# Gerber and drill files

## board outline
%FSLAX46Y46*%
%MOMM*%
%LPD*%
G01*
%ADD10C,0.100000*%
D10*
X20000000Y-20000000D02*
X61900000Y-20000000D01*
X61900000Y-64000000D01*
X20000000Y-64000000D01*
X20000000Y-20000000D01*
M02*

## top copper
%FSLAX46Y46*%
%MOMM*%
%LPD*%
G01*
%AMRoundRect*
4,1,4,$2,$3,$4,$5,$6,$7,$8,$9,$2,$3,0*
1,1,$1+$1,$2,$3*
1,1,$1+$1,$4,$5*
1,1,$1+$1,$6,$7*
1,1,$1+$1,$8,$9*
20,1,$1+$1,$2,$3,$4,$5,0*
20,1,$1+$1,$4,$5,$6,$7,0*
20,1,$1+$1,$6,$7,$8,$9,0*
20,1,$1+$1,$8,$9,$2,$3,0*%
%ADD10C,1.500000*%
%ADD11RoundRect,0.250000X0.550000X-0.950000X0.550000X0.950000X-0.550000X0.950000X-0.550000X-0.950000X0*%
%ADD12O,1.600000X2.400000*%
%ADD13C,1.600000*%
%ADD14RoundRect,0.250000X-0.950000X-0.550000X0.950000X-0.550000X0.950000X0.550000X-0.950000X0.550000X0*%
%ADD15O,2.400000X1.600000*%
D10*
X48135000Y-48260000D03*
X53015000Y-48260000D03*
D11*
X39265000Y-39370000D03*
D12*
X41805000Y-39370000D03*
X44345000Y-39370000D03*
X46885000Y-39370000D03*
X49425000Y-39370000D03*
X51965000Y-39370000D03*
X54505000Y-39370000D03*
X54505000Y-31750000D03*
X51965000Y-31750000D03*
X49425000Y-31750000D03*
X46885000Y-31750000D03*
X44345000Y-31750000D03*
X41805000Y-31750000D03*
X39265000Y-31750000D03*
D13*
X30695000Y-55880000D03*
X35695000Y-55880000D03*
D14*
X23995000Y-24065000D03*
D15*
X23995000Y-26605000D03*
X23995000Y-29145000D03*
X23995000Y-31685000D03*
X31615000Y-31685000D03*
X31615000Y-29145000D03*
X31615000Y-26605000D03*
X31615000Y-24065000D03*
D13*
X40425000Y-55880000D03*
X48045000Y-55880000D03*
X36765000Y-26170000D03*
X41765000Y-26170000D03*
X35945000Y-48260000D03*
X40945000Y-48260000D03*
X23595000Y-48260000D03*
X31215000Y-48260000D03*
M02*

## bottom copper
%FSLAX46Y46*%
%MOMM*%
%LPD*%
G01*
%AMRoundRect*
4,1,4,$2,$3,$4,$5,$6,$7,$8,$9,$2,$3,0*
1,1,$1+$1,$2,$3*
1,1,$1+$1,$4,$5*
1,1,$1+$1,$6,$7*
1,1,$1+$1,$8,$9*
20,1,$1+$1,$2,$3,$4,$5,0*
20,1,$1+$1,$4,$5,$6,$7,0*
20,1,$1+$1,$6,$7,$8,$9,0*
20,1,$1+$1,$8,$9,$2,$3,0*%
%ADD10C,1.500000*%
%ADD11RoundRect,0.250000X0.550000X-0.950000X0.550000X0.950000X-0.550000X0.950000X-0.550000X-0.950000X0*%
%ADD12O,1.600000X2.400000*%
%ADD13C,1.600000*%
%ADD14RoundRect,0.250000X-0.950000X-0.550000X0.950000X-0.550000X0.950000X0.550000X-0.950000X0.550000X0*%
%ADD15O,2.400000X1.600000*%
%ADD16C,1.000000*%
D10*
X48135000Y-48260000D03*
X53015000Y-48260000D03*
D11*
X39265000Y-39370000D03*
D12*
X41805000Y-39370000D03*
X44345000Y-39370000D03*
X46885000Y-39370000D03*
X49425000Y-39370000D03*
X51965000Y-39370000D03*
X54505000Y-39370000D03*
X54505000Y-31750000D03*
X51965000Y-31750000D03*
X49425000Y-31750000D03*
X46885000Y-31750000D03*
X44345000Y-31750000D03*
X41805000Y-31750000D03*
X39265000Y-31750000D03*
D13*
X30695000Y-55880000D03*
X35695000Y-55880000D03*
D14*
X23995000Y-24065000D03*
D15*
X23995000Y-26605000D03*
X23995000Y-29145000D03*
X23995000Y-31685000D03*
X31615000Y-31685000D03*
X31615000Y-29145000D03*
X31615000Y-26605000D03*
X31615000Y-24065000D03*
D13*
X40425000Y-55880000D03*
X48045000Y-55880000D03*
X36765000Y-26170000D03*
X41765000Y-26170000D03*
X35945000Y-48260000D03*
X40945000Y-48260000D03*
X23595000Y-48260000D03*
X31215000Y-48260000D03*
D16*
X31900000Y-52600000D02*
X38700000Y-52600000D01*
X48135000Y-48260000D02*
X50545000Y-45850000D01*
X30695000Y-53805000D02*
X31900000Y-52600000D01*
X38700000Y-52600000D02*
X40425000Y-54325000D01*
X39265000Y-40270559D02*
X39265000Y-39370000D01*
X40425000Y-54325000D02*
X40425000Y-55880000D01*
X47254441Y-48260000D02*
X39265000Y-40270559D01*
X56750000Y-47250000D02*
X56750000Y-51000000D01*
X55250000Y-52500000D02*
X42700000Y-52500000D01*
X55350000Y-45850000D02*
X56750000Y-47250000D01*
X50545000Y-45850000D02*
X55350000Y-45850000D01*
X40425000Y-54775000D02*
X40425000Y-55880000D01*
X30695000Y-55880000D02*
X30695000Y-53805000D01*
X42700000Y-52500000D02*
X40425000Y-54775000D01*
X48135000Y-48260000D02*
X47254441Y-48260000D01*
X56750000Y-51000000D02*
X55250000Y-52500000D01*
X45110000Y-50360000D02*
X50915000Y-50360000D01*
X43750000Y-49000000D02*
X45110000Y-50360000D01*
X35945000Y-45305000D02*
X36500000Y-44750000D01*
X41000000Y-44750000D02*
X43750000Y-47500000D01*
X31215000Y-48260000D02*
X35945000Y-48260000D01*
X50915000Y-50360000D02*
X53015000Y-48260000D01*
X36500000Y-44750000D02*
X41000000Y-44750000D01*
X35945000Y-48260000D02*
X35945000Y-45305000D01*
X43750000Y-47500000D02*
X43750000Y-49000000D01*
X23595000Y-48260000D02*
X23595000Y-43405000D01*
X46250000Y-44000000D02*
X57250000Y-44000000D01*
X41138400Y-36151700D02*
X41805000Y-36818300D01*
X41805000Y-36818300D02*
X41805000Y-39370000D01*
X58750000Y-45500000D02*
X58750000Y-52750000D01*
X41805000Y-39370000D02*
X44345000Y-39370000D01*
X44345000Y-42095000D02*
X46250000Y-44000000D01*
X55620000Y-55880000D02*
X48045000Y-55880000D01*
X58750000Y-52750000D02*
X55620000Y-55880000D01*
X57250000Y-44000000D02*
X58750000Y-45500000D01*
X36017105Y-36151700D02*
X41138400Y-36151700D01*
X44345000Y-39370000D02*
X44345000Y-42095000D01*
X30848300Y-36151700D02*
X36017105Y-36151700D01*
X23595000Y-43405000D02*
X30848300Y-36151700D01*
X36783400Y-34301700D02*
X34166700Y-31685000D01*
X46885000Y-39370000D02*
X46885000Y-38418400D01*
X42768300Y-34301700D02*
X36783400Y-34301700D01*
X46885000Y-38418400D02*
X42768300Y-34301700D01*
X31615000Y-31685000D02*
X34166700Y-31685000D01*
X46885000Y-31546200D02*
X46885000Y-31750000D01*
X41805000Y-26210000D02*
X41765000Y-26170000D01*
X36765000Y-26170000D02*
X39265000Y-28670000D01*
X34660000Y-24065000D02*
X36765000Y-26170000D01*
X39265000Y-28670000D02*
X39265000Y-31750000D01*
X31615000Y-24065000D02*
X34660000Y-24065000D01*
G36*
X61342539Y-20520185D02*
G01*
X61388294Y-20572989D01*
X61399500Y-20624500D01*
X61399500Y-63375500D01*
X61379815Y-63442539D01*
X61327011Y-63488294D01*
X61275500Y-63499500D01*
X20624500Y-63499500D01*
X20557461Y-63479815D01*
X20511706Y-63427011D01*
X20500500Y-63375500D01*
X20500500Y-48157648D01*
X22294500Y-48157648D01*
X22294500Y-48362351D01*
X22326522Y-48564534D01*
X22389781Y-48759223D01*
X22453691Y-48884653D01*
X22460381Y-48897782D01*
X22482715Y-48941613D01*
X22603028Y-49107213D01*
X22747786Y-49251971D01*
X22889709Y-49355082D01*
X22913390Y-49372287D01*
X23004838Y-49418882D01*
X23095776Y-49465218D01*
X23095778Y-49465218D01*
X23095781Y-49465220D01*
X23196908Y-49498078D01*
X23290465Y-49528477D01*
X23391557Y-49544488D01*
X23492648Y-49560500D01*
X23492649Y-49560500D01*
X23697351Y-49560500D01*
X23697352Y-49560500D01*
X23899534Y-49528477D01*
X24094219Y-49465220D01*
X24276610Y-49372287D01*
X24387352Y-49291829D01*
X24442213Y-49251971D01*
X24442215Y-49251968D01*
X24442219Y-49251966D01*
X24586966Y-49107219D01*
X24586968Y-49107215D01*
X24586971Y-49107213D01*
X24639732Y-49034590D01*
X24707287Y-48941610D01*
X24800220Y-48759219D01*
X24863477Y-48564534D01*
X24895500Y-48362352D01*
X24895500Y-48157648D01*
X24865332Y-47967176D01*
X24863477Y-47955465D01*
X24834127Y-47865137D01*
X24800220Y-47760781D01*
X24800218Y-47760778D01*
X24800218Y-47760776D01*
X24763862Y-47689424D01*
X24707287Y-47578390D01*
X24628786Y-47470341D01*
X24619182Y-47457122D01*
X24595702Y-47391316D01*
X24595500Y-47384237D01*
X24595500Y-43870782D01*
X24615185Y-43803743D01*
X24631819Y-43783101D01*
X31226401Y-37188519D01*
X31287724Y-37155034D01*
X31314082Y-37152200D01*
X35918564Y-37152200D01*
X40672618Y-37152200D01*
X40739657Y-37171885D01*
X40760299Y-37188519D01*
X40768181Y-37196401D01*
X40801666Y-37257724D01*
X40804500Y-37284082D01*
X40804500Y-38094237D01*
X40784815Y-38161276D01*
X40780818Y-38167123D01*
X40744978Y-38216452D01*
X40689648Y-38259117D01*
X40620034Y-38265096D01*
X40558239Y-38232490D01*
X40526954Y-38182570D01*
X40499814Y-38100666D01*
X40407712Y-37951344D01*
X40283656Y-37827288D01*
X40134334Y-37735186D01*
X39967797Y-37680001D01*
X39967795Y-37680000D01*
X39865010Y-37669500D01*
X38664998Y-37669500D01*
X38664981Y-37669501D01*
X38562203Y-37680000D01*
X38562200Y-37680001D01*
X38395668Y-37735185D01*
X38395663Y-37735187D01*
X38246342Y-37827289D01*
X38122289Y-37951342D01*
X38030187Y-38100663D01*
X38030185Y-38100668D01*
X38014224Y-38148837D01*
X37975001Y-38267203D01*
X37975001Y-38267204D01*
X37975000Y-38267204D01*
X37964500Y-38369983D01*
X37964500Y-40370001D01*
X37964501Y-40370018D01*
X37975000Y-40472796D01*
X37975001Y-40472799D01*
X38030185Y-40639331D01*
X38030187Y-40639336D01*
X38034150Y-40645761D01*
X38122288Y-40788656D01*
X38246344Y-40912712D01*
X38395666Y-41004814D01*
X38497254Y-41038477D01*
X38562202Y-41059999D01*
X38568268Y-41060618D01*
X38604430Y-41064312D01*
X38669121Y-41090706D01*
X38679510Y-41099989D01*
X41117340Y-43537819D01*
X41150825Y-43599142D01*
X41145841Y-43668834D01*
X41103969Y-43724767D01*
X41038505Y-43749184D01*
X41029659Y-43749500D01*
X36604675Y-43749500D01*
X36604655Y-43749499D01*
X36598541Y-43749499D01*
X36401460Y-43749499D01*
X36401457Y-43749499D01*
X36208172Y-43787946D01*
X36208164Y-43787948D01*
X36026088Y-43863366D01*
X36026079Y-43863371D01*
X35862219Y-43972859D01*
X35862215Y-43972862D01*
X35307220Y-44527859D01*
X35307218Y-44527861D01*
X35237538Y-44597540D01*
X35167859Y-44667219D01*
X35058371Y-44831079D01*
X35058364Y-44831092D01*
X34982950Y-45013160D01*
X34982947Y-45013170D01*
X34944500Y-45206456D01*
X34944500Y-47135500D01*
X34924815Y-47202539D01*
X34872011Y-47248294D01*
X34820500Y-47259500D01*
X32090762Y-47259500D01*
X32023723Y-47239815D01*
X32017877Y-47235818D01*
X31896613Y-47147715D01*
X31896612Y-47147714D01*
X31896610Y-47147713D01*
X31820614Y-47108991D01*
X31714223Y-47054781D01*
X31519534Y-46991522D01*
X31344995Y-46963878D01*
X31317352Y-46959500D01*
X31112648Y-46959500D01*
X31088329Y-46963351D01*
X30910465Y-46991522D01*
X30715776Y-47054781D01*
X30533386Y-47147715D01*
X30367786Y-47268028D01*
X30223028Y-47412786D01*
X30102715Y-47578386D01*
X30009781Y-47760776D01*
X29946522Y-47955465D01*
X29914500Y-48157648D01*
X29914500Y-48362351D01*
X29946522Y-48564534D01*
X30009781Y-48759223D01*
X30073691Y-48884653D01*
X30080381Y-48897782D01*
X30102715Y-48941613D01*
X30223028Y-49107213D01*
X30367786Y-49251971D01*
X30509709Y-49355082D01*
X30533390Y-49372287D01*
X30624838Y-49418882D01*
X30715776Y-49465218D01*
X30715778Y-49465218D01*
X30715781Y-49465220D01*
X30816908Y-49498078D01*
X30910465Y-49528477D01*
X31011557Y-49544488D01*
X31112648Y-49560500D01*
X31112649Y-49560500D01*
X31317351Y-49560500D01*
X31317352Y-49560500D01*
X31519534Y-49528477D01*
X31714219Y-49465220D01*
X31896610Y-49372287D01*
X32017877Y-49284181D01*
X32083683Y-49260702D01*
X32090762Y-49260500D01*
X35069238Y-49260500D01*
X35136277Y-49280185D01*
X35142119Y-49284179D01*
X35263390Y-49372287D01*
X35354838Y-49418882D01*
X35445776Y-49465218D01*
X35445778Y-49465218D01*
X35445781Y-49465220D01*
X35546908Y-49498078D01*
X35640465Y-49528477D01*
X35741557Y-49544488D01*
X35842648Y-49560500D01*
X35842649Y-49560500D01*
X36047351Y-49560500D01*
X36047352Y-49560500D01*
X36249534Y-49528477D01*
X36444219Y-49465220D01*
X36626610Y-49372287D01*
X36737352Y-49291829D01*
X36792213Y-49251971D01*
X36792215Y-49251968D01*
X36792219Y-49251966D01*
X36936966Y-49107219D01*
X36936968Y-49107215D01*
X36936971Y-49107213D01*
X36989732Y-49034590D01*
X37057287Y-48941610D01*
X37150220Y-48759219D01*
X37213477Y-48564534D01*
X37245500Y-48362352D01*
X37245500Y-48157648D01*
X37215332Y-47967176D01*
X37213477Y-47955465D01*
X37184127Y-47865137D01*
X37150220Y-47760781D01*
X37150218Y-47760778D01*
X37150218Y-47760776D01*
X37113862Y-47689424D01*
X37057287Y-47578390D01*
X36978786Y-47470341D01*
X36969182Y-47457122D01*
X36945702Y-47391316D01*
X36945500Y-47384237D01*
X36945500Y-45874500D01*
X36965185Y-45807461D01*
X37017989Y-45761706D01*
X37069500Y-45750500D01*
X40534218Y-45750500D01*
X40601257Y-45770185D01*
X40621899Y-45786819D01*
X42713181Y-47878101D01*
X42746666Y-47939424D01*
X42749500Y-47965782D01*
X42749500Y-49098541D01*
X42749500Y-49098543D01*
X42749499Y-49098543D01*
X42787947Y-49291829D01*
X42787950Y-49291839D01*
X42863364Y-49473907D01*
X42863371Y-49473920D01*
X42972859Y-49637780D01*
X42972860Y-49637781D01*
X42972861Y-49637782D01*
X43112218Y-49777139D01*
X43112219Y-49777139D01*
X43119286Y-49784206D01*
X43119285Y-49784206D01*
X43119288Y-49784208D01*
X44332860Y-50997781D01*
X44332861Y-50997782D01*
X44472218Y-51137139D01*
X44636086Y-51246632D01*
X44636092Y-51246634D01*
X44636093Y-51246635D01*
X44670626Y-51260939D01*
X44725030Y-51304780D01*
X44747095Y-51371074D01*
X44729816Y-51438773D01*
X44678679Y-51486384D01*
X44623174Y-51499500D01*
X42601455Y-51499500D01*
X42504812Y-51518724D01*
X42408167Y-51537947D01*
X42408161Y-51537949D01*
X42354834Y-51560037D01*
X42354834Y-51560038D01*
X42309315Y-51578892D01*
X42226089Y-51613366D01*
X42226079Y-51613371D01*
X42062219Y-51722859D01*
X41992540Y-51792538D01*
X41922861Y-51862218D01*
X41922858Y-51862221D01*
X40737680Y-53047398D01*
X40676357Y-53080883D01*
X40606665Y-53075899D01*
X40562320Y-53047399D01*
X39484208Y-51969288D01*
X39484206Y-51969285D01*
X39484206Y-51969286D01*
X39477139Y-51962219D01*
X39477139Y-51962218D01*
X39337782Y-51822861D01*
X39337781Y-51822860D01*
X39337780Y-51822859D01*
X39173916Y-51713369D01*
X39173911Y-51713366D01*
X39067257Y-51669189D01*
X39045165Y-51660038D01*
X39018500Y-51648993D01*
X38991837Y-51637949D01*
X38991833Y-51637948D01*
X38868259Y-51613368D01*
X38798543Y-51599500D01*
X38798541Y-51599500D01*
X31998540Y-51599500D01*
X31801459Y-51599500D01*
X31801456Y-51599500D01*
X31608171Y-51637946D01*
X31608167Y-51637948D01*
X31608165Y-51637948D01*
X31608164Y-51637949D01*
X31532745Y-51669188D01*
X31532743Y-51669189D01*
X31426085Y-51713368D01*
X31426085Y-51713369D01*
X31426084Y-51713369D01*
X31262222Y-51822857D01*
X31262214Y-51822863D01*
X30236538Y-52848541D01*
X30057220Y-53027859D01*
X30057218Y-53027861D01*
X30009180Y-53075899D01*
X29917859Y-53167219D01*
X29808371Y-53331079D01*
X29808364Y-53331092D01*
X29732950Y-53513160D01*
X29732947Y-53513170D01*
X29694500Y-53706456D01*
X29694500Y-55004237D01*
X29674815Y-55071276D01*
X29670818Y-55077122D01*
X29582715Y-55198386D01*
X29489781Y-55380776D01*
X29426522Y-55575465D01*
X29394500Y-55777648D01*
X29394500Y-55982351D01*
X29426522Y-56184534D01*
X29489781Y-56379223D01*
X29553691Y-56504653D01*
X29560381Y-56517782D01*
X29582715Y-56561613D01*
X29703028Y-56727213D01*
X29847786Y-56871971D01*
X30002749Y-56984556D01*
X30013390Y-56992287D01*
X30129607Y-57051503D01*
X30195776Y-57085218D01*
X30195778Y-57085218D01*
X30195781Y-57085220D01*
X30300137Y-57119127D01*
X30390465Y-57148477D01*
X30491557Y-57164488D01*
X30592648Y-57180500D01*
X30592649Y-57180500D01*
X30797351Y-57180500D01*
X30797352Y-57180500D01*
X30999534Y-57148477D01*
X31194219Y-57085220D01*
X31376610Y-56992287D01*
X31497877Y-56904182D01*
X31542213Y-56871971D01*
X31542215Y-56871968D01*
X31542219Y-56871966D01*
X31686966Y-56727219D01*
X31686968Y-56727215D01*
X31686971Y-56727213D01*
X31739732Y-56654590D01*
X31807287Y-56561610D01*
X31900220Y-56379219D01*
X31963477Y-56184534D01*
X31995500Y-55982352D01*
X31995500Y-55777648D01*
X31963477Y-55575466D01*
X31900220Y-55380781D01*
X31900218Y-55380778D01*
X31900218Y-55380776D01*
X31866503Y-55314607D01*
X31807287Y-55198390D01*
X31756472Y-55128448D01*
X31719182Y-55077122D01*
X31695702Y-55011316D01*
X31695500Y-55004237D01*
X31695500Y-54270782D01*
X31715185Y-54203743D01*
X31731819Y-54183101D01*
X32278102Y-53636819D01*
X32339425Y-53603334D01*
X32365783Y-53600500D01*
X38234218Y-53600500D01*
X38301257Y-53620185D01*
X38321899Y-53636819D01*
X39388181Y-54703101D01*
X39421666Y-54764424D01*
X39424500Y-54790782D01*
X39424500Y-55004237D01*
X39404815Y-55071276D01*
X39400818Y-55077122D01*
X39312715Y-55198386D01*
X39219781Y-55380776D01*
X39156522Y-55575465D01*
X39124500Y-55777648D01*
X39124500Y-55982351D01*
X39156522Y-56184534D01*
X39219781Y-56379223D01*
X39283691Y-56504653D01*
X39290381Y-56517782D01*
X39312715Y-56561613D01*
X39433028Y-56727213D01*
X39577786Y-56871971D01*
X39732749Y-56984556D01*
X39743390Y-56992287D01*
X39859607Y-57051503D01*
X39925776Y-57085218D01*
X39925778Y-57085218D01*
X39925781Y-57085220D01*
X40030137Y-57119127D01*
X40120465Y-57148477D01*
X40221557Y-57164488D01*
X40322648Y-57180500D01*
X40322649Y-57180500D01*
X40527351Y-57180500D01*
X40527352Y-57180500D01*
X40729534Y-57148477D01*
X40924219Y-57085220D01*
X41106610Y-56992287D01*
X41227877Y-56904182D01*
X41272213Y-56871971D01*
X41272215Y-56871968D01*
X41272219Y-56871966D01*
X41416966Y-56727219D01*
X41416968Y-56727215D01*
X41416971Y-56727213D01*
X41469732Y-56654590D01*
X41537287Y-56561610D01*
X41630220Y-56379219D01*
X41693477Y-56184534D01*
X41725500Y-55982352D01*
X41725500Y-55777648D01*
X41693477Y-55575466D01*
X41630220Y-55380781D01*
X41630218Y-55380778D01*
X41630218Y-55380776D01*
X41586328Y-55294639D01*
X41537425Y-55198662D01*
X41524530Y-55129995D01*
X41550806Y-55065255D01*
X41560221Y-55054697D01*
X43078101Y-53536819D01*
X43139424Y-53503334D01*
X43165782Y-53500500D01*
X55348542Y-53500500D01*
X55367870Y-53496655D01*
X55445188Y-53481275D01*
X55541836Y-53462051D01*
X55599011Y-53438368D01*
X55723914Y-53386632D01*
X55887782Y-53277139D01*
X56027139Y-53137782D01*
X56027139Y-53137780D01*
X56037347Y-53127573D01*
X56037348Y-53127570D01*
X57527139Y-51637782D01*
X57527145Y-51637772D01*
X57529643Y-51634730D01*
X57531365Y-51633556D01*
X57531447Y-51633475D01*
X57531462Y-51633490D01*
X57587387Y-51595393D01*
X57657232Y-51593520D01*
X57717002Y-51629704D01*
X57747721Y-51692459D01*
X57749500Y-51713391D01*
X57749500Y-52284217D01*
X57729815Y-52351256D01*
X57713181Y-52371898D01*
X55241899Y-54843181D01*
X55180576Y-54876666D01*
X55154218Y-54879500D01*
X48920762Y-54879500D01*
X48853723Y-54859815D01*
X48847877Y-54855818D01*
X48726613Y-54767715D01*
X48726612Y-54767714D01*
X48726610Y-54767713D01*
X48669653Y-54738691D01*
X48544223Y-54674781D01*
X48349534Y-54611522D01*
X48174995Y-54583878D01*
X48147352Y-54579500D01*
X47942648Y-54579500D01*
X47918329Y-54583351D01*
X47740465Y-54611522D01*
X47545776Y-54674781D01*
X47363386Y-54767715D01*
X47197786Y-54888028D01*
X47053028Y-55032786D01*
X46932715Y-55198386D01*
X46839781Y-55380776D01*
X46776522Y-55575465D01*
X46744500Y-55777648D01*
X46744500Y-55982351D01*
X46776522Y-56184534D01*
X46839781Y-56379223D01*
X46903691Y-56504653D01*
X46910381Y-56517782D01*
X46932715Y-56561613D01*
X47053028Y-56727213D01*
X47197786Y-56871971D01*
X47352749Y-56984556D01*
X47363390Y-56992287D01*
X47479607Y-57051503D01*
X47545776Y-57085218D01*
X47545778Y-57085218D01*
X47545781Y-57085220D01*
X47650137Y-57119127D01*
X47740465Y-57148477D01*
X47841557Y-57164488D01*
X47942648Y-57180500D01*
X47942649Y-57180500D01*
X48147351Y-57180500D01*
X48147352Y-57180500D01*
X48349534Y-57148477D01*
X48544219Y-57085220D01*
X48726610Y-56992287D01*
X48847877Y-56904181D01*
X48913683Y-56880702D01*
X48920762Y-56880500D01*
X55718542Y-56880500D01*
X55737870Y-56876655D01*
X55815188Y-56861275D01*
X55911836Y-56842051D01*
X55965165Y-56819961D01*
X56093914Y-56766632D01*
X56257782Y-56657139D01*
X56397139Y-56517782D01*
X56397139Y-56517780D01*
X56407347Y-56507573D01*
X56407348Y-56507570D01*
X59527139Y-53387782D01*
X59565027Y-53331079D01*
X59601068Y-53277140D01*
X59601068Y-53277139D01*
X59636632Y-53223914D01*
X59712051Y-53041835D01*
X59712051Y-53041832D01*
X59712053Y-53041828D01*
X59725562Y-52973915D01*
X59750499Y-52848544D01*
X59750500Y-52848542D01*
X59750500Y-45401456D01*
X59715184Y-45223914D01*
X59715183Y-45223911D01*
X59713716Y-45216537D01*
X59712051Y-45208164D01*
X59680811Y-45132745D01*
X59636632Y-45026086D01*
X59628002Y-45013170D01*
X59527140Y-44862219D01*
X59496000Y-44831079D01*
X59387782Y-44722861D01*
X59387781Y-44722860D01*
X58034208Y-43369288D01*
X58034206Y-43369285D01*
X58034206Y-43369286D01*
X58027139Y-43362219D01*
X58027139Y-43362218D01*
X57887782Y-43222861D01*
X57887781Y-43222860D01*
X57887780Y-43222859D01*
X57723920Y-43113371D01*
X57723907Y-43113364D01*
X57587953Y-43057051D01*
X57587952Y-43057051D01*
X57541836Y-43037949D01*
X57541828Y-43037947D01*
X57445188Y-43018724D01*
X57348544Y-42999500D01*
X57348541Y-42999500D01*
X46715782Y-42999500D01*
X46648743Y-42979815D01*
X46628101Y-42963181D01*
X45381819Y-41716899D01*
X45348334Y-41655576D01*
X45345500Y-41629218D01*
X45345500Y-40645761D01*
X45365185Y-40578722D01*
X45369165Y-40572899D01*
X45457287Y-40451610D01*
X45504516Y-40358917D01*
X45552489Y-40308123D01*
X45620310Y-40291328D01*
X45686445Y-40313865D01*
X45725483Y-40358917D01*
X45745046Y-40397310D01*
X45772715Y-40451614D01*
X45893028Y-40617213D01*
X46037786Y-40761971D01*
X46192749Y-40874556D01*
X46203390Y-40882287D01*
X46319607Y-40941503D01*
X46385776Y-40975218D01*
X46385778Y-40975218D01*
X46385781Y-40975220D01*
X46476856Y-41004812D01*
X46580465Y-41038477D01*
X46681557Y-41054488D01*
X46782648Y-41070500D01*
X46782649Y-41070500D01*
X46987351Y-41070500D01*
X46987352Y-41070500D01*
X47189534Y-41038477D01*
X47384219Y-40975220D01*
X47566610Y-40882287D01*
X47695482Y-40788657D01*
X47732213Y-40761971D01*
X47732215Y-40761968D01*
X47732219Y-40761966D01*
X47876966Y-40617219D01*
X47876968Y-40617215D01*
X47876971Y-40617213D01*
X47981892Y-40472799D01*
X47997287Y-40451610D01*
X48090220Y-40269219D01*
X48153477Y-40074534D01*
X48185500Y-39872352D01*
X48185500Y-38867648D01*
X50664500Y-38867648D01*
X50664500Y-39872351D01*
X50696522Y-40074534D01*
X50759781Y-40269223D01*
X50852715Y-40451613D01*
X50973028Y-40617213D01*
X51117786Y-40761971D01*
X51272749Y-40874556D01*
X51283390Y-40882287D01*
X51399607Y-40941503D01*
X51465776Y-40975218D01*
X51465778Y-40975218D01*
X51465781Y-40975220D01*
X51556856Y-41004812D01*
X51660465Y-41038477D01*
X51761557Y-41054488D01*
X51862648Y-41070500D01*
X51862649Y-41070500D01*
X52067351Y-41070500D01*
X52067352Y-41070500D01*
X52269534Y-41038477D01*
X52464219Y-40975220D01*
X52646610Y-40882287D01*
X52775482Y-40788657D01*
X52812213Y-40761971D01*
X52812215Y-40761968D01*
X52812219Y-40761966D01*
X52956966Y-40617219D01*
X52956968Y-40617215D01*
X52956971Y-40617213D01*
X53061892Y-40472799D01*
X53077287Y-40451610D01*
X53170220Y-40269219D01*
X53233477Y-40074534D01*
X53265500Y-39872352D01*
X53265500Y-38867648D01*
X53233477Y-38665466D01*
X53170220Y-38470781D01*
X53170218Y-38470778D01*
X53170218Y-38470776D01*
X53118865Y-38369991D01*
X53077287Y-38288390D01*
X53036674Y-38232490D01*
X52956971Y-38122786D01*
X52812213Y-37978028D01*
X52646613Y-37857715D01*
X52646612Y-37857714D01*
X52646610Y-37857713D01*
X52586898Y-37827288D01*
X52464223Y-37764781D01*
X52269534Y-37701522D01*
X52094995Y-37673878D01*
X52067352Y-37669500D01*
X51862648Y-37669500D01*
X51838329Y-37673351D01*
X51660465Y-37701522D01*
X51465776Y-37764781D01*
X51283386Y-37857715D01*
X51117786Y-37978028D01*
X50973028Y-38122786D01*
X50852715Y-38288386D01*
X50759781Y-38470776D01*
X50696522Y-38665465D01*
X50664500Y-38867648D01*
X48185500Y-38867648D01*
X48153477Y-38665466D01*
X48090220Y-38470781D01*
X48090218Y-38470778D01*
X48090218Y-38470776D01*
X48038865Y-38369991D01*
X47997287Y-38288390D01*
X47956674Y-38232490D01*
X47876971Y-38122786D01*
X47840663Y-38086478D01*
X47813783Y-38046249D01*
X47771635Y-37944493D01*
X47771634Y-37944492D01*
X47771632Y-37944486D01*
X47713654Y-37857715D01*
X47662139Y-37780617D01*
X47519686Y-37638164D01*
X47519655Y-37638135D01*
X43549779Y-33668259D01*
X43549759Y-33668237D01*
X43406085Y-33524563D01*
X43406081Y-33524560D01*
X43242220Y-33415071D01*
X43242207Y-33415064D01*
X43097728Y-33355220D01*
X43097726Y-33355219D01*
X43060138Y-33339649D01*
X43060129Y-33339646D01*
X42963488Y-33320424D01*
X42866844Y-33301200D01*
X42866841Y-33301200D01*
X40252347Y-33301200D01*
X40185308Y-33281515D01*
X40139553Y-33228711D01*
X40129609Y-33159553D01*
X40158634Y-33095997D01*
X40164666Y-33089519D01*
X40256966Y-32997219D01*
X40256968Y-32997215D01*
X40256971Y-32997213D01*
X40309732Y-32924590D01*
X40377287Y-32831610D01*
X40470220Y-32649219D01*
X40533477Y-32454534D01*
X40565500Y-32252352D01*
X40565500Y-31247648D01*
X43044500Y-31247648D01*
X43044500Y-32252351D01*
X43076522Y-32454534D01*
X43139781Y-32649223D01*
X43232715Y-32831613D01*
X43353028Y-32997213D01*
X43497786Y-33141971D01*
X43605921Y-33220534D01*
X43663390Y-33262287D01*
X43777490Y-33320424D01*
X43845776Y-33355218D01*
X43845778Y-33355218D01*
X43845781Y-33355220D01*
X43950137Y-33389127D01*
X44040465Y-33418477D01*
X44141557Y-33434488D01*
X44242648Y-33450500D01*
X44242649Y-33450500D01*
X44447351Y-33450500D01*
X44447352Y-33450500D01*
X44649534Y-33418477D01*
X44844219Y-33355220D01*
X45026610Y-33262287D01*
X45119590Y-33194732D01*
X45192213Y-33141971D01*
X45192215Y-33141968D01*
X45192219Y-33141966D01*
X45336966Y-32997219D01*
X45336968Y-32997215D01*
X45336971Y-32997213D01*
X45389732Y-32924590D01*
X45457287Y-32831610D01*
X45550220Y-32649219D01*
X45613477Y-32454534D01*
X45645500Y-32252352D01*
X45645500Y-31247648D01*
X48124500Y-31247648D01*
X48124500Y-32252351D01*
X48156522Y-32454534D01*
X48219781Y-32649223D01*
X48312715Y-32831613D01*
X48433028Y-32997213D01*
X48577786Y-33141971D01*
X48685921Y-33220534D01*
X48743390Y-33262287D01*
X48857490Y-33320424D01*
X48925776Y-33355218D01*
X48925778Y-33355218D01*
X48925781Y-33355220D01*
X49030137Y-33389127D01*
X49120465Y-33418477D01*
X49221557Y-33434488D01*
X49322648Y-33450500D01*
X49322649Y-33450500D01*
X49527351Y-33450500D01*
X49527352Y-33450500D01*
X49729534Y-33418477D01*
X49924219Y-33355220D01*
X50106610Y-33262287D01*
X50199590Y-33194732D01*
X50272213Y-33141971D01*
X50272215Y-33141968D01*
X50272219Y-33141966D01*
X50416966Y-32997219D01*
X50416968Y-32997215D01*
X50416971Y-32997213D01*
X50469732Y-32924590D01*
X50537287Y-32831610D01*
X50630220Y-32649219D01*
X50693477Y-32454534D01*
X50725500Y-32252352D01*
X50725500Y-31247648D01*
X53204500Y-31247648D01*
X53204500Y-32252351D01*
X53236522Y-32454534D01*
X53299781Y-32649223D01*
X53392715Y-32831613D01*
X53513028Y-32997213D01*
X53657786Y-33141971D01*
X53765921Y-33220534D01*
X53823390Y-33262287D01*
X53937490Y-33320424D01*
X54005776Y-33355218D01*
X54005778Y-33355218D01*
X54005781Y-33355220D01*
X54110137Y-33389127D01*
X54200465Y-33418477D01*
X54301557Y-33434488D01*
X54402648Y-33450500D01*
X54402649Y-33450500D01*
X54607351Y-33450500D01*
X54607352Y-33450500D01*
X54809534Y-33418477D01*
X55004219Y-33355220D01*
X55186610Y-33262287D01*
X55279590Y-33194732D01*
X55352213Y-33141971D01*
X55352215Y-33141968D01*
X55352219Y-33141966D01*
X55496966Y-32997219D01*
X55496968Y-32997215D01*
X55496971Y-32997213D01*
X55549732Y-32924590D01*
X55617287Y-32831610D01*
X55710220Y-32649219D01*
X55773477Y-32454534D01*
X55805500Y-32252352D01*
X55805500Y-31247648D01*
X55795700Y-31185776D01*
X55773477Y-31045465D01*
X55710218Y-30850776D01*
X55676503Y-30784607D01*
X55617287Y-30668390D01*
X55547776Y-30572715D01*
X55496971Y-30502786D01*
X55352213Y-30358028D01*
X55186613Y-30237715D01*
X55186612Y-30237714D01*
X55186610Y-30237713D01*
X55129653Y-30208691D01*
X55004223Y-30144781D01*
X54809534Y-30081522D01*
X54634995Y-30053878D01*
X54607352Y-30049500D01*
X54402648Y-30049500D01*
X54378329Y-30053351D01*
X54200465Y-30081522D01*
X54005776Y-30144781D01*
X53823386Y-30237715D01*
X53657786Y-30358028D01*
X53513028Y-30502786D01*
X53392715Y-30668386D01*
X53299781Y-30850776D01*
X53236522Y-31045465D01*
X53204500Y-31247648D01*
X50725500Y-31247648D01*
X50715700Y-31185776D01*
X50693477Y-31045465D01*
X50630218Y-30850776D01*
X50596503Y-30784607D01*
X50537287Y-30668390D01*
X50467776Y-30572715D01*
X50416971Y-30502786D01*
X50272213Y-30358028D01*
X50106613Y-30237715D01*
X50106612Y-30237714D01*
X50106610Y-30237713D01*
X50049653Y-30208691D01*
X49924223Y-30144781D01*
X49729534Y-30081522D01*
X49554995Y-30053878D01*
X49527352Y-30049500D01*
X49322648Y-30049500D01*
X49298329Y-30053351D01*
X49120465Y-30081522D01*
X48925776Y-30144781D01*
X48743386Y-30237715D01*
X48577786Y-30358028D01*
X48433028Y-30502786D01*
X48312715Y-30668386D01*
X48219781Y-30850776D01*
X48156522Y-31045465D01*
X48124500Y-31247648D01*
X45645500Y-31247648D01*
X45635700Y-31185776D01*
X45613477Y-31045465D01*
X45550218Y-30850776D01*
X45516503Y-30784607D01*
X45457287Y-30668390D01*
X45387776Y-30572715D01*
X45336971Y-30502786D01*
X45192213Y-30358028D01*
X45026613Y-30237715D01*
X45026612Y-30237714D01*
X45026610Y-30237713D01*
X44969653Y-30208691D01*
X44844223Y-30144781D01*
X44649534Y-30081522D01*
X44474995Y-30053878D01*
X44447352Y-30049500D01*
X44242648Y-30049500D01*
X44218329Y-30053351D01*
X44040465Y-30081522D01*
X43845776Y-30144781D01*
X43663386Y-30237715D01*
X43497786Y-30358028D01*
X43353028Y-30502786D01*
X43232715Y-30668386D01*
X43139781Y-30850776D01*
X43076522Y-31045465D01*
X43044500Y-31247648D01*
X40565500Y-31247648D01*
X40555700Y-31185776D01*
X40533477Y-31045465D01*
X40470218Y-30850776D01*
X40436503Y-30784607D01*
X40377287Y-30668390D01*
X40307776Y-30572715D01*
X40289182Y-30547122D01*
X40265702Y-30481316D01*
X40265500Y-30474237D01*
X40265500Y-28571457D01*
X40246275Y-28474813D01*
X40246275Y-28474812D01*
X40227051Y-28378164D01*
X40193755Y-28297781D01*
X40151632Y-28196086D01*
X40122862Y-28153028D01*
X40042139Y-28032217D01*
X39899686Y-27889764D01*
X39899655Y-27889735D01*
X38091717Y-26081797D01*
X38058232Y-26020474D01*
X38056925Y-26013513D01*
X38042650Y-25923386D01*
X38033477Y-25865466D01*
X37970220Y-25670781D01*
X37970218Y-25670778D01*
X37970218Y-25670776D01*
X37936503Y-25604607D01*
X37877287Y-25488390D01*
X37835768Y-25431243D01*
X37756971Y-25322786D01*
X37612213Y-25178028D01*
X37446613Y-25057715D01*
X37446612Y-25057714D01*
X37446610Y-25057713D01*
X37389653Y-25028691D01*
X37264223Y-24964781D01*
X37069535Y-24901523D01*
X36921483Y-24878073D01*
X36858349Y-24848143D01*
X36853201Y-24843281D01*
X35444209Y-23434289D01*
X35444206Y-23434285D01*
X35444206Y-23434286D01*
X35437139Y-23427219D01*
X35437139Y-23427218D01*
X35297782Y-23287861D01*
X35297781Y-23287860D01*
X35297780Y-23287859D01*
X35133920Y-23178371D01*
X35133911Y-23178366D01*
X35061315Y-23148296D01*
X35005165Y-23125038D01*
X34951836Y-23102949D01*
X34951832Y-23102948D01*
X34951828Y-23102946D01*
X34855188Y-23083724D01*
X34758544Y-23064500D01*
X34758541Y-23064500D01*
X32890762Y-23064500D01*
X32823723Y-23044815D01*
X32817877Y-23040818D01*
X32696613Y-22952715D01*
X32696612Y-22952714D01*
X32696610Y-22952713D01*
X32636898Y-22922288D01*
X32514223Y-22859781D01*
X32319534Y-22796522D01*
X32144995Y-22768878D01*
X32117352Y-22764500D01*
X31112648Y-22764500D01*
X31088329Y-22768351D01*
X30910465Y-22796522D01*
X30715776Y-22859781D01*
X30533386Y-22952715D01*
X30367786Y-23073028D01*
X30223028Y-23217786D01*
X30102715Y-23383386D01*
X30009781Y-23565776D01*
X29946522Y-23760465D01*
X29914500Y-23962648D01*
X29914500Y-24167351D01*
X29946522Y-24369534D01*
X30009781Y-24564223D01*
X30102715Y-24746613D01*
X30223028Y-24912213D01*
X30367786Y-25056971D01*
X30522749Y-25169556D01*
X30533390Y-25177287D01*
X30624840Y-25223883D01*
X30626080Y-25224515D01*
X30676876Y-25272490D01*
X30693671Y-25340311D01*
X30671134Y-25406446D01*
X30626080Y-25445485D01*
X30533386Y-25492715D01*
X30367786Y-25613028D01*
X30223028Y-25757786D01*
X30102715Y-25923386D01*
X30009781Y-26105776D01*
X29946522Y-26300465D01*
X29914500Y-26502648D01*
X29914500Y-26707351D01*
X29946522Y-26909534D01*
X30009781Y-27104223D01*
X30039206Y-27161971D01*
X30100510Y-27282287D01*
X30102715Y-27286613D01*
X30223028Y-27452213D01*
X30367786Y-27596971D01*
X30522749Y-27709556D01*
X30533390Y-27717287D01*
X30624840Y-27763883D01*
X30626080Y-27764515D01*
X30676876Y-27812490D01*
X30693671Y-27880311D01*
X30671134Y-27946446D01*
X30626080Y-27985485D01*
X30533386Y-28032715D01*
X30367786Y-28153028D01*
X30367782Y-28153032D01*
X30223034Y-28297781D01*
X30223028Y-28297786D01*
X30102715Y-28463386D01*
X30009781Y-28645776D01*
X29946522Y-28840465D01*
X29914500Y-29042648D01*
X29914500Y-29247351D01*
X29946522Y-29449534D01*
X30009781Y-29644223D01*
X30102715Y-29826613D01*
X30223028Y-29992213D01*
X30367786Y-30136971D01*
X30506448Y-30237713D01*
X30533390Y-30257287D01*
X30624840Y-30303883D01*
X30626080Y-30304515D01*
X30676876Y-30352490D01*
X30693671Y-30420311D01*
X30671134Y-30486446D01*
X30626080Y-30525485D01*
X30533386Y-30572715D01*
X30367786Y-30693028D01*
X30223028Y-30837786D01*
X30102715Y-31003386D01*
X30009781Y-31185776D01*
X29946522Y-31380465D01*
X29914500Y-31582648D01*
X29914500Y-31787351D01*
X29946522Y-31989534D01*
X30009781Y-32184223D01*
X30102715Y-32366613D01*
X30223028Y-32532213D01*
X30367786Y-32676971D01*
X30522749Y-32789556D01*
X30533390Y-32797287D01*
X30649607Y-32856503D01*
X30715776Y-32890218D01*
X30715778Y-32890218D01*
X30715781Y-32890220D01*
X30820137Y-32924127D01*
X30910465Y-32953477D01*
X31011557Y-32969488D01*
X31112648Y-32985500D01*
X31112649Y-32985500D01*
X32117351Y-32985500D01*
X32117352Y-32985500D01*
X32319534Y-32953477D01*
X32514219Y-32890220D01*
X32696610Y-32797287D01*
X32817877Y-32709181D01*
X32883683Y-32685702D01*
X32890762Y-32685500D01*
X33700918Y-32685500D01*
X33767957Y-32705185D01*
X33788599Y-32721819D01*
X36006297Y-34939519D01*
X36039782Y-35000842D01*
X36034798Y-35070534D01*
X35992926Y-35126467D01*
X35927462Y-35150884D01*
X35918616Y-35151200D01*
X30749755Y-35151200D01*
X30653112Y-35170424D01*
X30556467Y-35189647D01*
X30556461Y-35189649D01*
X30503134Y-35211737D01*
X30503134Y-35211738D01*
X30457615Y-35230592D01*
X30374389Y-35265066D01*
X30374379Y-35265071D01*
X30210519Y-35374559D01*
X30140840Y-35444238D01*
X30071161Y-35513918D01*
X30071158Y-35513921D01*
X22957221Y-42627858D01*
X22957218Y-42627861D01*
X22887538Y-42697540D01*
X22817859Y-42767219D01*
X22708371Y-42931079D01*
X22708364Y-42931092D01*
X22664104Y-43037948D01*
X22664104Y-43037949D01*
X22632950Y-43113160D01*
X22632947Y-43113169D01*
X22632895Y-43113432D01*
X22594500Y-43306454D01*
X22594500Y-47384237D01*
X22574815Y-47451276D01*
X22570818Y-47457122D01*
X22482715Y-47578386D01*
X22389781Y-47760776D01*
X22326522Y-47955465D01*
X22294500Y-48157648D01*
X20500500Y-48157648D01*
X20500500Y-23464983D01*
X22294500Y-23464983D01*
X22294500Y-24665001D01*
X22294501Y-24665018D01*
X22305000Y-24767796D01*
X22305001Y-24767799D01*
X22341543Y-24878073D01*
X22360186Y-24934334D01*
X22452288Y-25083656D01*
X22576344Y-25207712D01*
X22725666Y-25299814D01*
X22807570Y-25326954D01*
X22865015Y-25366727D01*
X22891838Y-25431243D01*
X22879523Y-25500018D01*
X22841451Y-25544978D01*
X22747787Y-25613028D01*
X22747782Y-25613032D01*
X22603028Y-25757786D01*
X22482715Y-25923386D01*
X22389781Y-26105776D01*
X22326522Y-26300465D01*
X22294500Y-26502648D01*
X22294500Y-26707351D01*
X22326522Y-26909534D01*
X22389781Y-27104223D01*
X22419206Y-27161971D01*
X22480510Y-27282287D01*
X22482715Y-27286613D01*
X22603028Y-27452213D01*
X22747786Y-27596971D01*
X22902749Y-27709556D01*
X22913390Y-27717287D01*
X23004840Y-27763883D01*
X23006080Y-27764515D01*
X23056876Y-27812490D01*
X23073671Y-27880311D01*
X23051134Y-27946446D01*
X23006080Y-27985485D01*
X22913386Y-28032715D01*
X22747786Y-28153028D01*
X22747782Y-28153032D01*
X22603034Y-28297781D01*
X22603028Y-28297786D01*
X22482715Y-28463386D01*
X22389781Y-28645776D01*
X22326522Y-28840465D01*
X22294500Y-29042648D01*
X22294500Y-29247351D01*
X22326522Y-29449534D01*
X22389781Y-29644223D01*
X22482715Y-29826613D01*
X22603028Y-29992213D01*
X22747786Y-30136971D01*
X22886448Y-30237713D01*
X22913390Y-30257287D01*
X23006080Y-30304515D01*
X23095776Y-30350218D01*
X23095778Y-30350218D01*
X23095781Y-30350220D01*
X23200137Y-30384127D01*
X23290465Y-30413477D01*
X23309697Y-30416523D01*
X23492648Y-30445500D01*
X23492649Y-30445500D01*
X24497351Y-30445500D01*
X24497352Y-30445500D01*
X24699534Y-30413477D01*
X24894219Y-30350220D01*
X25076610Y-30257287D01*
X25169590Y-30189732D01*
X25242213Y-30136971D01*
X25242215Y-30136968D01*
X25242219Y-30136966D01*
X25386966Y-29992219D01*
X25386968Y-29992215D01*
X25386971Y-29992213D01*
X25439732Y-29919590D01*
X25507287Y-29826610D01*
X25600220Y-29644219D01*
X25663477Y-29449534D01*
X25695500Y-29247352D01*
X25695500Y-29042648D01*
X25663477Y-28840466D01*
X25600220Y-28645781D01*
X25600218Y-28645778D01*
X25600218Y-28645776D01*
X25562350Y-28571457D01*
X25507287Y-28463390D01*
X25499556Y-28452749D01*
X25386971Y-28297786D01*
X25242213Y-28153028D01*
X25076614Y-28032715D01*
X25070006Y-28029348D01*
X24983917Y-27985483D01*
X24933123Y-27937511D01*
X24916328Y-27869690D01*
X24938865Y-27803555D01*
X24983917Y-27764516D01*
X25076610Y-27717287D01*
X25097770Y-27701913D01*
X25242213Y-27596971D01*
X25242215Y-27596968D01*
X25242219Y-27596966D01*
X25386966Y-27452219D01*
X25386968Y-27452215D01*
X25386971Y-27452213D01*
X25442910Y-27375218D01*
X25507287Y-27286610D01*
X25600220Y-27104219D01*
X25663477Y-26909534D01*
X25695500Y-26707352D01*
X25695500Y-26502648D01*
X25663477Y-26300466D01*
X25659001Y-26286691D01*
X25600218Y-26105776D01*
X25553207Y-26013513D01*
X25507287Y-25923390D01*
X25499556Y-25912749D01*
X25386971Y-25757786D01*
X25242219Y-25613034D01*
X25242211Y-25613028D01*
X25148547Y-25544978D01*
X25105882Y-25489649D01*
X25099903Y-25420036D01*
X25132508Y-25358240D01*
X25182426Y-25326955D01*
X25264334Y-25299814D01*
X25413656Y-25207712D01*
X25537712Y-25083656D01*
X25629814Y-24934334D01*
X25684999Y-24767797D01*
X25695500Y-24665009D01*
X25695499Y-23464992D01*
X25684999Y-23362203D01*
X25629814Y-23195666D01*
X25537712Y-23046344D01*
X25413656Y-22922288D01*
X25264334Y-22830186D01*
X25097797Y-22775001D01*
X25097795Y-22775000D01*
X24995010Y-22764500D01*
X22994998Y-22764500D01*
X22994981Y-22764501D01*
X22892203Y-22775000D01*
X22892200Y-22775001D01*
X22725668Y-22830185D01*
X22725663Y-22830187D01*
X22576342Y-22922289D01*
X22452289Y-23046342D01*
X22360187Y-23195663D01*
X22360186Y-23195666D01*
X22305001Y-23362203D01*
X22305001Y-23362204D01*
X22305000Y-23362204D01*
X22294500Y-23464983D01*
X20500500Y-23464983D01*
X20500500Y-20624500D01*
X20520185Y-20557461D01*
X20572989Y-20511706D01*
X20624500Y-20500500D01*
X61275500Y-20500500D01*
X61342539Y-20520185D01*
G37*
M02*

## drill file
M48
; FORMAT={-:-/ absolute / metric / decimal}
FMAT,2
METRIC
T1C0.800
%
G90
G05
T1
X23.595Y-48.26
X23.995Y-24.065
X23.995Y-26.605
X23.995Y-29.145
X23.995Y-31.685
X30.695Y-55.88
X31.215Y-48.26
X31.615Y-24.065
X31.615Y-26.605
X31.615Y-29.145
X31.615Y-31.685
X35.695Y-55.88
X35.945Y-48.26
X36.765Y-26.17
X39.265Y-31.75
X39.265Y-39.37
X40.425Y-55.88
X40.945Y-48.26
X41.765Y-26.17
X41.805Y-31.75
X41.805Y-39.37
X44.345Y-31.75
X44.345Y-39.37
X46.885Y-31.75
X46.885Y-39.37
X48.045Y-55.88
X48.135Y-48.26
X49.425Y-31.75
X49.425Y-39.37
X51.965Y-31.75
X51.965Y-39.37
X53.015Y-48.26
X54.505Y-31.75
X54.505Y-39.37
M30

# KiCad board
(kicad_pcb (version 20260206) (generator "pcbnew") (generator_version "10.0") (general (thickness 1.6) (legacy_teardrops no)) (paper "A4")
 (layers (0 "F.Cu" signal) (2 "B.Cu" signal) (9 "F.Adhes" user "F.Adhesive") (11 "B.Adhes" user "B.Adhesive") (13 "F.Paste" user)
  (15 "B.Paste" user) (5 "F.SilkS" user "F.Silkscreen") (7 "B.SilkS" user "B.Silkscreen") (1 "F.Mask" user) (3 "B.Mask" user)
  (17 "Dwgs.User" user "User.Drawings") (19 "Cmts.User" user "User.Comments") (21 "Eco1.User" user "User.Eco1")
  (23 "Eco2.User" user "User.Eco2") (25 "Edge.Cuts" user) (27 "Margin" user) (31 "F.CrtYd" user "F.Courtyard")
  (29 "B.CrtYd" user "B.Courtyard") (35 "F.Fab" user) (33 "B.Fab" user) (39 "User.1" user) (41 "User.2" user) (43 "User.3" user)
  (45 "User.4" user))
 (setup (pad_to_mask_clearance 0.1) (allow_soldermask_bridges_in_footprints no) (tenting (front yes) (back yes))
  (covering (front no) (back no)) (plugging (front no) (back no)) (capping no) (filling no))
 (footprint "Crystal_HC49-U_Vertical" (layer "F.Cu") (at 48.135 48.26)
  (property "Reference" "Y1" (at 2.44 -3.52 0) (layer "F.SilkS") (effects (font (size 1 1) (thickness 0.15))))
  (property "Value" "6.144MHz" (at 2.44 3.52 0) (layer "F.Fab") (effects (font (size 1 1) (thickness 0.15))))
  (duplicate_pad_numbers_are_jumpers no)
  (pad "1" thru_hole circle (at 0 0) (size 1.5 1.5) (drill 0.8) (layers "*.Cu" "*.Mask") (remove_unused_layers no) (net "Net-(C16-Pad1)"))
  (pad "2" thru_hole circle (at 4.88 0) (size 1.5 1.5) (drill 0.8) (layers "*.Cu" "*.Mask") (remove_unused_layers no) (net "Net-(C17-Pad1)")))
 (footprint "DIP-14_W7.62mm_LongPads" (layer "F.Cu") (at 39.265 39.37 90)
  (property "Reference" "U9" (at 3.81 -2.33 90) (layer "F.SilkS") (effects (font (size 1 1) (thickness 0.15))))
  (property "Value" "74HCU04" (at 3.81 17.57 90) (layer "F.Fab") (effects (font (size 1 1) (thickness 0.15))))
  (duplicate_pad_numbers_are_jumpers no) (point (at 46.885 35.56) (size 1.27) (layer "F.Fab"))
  (pad "1" thru_hole roundrect (at 0 0 90) (size 2.4 1.6) (drill 0.8) (layers "*.Cu" "*.Mask") (remove_unused_layers no)
   (roundrect_rratio 0.15625) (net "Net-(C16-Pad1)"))
  (pad "2" thru_hole oval (at 0 2.54 90) (size 2.4 1.6) (drill 0.8) (layers "*.Cu" "*.Mask") (remove_unused_layers no)
   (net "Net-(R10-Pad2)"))
  (pad "3" thru_hole oval (at 0 5.08 90) (size 2.4 1.6) (drill 0.8) (layers "*.Cu" "*.Mask") (remove_unused_layers no)
   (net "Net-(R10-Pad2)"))
  (pad "4" thru_hole oval (at 0 7.62 90) (size 2.4 1.6) (drill 0.8) (layers "*.Cu" "*.Mask") (remove_unused_layers no)
   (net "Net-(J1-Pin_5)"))
  (pad "5" thru_hole oval (at 0 10.16 90) (size 2.4 1.6) (drill 0.8) (layers "*.Cu" "*.Mask") (remove_unused_layers no) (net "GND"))
  (pad "6" thru_hole oval (at 0 12.7 90) (size 2.4 1.6) (drill 0.8) (layers "*.Cu" "*.Mask") (remove_unused_layers no))
  (pad "7" thru_hole oval (at 0 15.24 90) (size 2.4 1.6) (drill 0.8) (layers "*.Cu" "*.Mask") (remove_unused_layers no) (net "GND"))
  (pad "8" thru_hole oval (at 7.62 15.24 90) (size 2.4 1.6) (drill 0.8) (layers "*.Cu" "*.Mask") (remove_unused_layers no))
  (pad "9" thru_hole oval (at 7.62 12.7 90) (size 2.4 1.6) (drill 0.8) (layers "*.Cu" "*.Mask") (remove_unused_layers no) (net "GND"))
  (pad "10" thru_hole oval (at 7.62 10.16 90) (size 2.4 1.6) (drill 0.8) (layers "*.Cu" "*.Mask") (remove_unused_layers no))
  (pad "11" thru_hole oval (at 7.62 7.62 90) (size 2.4 1.6) (drill 0.8) (layers "*.Cu" "*.Mask") (remove_unused_layers no) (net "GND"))
  (pad "12" thru_hole oval (at 7.62 5.08 90) (size 2.4 1.6) (drill 0.8) (layers "*.Cu" "*.Mask") (remove_unused_layers no))
  (pad "13" thru_hole oval (at 7.62 2.54 90) (size 2.4 1.6) (drill 0.8) (layers "*.Cu" "*.Mask") (remove_unused_layers no) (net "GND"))
  (pad "14" thru_hole oval (at 7.62 0 90) (size 2.4 1.6) (drill 0.8) (layers "*.Cu" "*.Mask") (remove_unused_layers no) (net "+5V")))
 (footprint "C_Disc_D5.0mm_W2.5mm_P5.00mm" (layer "F.Cu") (at 30.695 55.88)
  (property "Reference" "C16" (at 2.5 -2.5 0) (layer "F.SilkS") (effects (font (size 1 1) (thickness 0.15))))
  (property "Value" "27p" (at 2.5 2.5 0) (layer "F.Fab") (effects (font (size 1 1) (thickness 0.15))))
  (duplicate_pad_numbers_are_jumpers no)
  (pad "1" thru_hole circle (at 0 0) (size 1.6 1.6) (drill 0.8) (layers "*.Cu" "*.Mask") (remove_unused_layers no) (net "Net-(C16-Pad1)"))
  (pad "2" thru_hole circle (at 5 0) (size 1.6 1.6) (drill 0.8) (layers "*.Cu" "*.Mask") (remove_unused_layers no) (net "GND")))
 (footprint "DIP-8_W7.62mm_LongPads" (layer "F.Cu") (at 23.995 24.065)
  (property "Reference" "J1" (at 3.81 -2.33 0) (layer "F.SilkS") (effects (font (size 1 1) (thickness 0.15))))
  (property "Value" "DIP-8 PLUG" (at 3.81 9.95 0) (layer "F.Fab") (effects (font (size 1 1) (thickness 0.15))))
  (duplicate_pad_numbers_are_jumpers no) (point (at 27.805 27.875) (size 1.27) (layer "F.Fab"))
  (pad "1" thru_hole roundrect (at 0 0) (size 2.4 1.6) (drill 0.8) (layers "*.Cu" "*.Mask") (remove_unused_layers no)
   (roundrect_rratio 0.15625))
  (pad "2" thru_hole oval (at 0 2.54) (size 2.4 1.6) (drill 0.8) (layers "*.Cu" "*.Mask") (remove_unused_layers no))
  (pad "3" thru_hole oval (at 0 5.08) (size 2.4 1.6) (drill 0.8) (layers "*.Cu" "*.Mask") (remove_unused_layers no))
  (pad "4" thru_hole oval (at 0 7.62) (size 2.4 1.6) (drill 0.8) (layers "*.Cu" "*.Mask") (remove_unused_layers no) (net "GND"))
  (pad "5" thru_hole oval (at 7.62 7.62) (size 2.4 1.6) (drill 0.8) (layers "*.Cu" "*.Mask") (remove_unused_layers no)
   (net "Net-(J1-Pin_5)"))
  (pad "6" thru_hole oval (at 7.62 5.08) (size 2.4 1.6) (drill 0.8) (layers "*.Cu" "*.Mask") (remove_unused_layers no))
  (pad "7" thru_hole oval (at 7.62 2.54) (size 2.4 1.6) (drill 0.8) (layers "*.Cu" "*.Mask") (remove_unused_layers no))
  (pad "8" thru_hole oval (at 7.62 0) (size 2.4 1.6) (drill 0.8) (layers "*.Cu" "*.Mask") (remove_unused_layers no) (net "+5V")))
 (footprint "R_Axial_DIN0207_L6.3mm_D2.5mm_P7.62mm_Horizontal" (layer "F.Cu") (at 40.425 55.88)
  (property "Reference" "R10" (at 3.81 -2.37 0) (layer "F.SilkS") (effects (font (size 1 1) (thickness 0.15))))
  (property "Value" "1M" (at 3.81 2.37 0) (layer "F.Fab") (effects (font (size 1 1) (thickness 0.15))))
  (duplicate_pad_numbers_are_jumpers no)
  (pad "1" thru_hole circle (at 0 0) (size 1.6 1.6) (drill 0.8) (layers "*.Cu" "*.Mask") (remove_unused_layers no) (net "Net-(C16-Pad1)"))
  (pad "2" thru_hole circle (at 7.62 0) (size 1.6 1.6) (drill 0.8) (layers "*.Cu" "*.Mask") (remove_unused_layers no) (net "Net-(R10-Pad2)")))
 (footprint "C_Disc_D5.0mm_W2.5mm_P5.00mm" (layer "F.Cu") (at 36.765 26.17)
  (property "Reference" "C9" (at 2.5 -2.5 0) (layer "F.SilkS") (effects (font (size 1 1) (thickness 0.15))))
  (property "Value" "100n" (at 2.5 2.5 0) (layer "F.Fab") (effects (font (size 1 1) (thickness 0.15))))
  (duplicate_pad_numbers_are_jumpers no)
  (pad "1" thru_hole circle (at 0 0) (size 1.6 1.6) (drill 0.8) (layers "*.Cu" "*.Mask") (remove_unused_layers no) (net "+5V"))
  (pad "2" thru_hole circle (at 5 0) (size 1.6 1.6) (drill 0.8) (layers "*.Cu" "*.Mask") (remove_unused_layers no) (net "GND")))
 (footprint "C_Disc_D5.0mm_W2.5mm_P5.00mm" (layer "F.Cu") (at 35.945 48.26)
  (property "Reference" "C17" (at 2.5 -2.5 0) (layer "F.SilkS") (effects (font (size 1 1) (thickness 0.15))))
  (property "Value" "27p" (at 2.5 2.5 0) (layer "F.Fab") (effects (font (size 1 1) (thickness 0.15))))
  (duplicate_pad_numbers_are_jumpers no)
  (pad "1" thru_hole circle (at 0 0) (size 1.6 1.6) (drill 0.8) (layers "*.Cu" "*.Mask") (remove_unused_layers no) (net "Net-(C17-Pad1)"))
  (pad "2" thru_hole circle (at 5 0) (size 1.6 1.6) (drill 0.8) (layers "*.Cu" "*.Mask") (remove_unused_layers no) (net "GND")))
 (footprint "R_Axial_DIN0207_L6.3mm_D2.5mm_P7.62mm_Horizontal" (layer "F.Cu") (at 23.595 48.26)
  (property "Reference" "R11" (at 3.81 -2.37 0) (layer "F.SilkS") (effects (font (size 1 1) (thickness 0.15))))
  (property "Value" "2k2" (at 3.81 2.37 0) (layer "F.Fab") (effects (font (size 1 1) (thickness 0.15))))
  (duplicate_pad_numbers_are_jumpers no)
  (pad "1" thru_hole circle (at 0 0) (size 1.6 1.6) (drill 0.8) (layers "*.Cu" "*.Mask") (remove_unused_layers no) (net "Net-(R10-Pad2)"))
  (pad "2" thru_hole circle (at 7.62 0) (size 1.6 1.6) (drill 0.8) (layers "*.Cu" "*.Mask") (remove_unused_layers no) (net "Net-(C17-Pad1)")))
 (gr_rect (start 20 20) (end 61.9 64) (stroke (width 0.1) (type default)) (fill no) (layer "Edge.Cuts"))
 (segment (start 31.9 52.6) (end 38.7 52.6) (width 1) (layer "B.Cu") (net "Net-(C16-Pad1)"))
 (segment (start 48.135 48.26) (end 50.545 45.85) (width 1) (layer "B.Cu") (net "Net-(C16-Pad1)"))
 (segment (start 30.695 53.805) (end 31.9 52.6) (width 1) (layer "B.Cu") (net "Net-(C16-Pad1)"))
 (segment (start 38.7 52.6) (end 40.425 54.325) (width 1) (layer "B.Cu") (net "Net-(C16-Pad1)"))
 (segment (start 39.265 40.270559) (end 39.265 39.37) (width 1) (layer "B.Cu") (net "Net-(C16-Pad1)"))
 (segment (start 40.425 54.325) (end 40.425 55.88) (width 1) (layer "B.Cu") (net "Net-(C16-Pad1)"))
 (segment (start 47.254441 48.26) (end 39.265 40.270559) (width 1) (layer "B.Cu") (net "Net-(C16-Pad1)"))
 (segment (start 56.75 47.25) (end 56.75 51) (width 1) (layer "B.Cu") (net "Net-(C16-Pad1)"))
 (segment (start 55.25 52.5) (end 42.7 52.5) (width 1) (layer "B.Cu") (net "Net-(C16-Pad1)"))
 (segment (start 55.35 45.85) (end 56.75 47.25) (width 1) (layer "B.Cu") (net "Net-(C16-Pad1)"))
 (segment (start 50.545 45.85) (end 55.35 45.85) (width 1) (layer "B.Cu") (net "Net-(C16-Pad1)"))
 (segment (start 40.425 54.775) (end 40.425 55.88) (width 1) (layer "B.Cu") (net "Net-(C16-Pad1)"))
 (segment (start 30.695 55.88) (end 30.695 53.805) (width 1) (layer "B.Cu") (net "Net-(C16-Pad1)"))
 (segment (start 42.7 52.5) (end 40.425 54.775) (width 1) (layer "B.Cu") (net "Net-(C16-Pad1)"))
 (segment (start 48.135 48.26) (end 47.254441 48.26) (width 1) (layer "B.Cu") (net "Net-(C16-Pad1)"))
 (segment (start 56.75 51) (end 55.25 52.5) (width 1) (layer "B.Cu") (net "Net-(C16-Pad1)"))
 (segment (start 45.11 50.36) (end 50.915 50.36) (width 1) (layer "B.Cu") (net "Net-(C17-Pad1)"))
 (segment (start 43.75 49) (end 45.11 50.36) (width 1) (layer "B.Cu") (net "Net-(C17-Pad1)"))
 (segment (start 35.945 45.305) (end 36.5 44.75) (width 1) (layer "B.Cu") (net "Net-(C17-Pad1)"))
 (segment (start 41 44.75) (end 43.75 47.5) (width 1) (layer "B.Cu") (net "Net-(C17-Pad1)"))
 (segment (start 31.215 48.26) (end 35.945 48.26) (width 1) (layer "B.Cu") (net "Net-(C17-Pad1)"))
 (segment (start 50.915 50.36) (end 53.015 48.26) (width 1) (layer "B.Cu") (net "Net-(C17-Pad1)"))
 (segment (start 36.5 44.75) (end 41 44.75) (width 1) (layer "B.Cu") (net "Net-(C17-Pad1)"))
 (segment (start 35.945 48.26) (end 35.945 45.305) (width 1) (layer "B.Cu") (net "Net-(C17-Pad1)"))
 (segment (start 43.75 47.5) (end 43.75 49) (width 1) (layer "B.Cu") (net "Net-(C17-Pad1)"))
 (segment (start 23.595 48.26) (end 23.595 43.405) (width 1) (layer "B.Cu") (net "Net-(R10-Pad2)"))
 (segment (start 46.25 44) (end 57.25 44) (width 1) (layer "B.Cu") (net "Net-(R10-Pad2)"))
 (segment (start 41.1384 36.1517) (end 41.805 36.8183) (width 1) (layer "B.Cu") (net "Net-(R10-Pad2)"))
 (segment (start 41.805 36.8183) (end 41.805 39.37) (width 1) (layer "B.Cu") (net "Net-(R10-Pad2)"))
 (segment (start 58.75 45.5) (end 58.75 52.75) (width 1) (layer "B.Cu") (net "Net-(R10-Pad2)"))
 (segment (start 41.805 39.37) (end 44.345 39.37) (width 1) (layer "B.Cu") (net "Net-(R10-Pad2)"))
 (segment (start 44.345 42.095) (end 46.25 44) (width 1) (layer "B.Cu") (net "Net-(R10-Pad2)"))
 (segment (start 55.62 55.88) (end 48.045 55.88) (width 1) (layer "B.Cu") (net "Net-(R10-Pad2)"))
 (segment (start 58.75 52.75) (end 55.62 55.88) (width 1) (layer "B.Cu") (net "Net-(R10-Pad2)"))
 (segment (start 57.25 44) (end 58.75 45.5) (width 1) (layer "B.Cu") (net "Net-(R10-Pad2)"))
 (segment (start 36.017105 36.1517) (end 41.1384 36.1517) (width 1) (layer "B.Cu") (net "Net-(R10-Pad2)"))
 (segment (start 44.345 39.37) (end 44.345 42.095) (width 1) (layer "B.Cu") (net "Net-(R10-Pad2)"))
 (segment (start 30.8483 36.1517) (end 36.017105 36.1517) (width 1) (layer "B.Cu") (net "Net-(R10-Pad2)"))
 (segment (start 23.595 43.405) (end 30.8483 36.1517) (width 1) (layer "B.Cu") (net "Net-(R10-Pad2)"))
 (segment (start 36.7834 34.3017) (end 34.1667 31.685) (width 1) (layer "B.Cu") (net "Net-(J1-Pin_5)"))
 (segment (start 46.885 39.37) (end 46.885 38.4184) (width 1) (layer "B.Cu") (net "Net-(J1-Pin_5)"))
 (segment (start 42.7683 34.3017) (end 36.7834 34.3017) (width 1) (layer "B.Cu") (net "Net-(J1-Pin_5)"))
 (segment (start 46.885 38.4184) (end 42.7683 34.3017) (width 1) (layer "B.Cu") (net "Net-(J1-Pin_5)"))
 (segment (start 31.615 31.685) (end 34.1667 31.685) (width 1) (layer "B.Cu") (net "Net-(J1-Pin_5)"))
 (segment (start 46.885 31.5462) (end 46.885 31.75) (width 1) (layer "B.Cu") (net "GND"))
 (segment (start 41.805 26.21) (end 41.765 26.17) (width 1) (layer "B.Cu") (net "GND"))
 (segment (start 36.765 26.17) (end 39.265 28.67) (width 1) (layer "B.Cu") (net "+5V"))
 (segment (start 34.66 24.065) (end 36.765 26.17) (width 1) (layer "B.Cu") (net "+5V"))
 (segment (start 39.265 28.67) (end 39.265 31.75) (width 1) (layer "B.Cu") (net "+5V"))
 (segment (start 31.615 24.065) (end 34.66 24.065) (width 1) (layer "B.Cu") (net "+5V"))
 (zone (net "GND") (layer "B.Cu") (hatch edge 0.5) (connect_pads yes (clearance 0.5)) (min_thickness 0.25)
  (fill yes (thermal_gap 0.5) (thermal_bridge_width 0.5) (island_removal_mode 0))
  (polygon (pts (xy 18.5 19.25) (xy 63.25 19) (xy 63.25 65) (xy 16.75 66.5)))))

